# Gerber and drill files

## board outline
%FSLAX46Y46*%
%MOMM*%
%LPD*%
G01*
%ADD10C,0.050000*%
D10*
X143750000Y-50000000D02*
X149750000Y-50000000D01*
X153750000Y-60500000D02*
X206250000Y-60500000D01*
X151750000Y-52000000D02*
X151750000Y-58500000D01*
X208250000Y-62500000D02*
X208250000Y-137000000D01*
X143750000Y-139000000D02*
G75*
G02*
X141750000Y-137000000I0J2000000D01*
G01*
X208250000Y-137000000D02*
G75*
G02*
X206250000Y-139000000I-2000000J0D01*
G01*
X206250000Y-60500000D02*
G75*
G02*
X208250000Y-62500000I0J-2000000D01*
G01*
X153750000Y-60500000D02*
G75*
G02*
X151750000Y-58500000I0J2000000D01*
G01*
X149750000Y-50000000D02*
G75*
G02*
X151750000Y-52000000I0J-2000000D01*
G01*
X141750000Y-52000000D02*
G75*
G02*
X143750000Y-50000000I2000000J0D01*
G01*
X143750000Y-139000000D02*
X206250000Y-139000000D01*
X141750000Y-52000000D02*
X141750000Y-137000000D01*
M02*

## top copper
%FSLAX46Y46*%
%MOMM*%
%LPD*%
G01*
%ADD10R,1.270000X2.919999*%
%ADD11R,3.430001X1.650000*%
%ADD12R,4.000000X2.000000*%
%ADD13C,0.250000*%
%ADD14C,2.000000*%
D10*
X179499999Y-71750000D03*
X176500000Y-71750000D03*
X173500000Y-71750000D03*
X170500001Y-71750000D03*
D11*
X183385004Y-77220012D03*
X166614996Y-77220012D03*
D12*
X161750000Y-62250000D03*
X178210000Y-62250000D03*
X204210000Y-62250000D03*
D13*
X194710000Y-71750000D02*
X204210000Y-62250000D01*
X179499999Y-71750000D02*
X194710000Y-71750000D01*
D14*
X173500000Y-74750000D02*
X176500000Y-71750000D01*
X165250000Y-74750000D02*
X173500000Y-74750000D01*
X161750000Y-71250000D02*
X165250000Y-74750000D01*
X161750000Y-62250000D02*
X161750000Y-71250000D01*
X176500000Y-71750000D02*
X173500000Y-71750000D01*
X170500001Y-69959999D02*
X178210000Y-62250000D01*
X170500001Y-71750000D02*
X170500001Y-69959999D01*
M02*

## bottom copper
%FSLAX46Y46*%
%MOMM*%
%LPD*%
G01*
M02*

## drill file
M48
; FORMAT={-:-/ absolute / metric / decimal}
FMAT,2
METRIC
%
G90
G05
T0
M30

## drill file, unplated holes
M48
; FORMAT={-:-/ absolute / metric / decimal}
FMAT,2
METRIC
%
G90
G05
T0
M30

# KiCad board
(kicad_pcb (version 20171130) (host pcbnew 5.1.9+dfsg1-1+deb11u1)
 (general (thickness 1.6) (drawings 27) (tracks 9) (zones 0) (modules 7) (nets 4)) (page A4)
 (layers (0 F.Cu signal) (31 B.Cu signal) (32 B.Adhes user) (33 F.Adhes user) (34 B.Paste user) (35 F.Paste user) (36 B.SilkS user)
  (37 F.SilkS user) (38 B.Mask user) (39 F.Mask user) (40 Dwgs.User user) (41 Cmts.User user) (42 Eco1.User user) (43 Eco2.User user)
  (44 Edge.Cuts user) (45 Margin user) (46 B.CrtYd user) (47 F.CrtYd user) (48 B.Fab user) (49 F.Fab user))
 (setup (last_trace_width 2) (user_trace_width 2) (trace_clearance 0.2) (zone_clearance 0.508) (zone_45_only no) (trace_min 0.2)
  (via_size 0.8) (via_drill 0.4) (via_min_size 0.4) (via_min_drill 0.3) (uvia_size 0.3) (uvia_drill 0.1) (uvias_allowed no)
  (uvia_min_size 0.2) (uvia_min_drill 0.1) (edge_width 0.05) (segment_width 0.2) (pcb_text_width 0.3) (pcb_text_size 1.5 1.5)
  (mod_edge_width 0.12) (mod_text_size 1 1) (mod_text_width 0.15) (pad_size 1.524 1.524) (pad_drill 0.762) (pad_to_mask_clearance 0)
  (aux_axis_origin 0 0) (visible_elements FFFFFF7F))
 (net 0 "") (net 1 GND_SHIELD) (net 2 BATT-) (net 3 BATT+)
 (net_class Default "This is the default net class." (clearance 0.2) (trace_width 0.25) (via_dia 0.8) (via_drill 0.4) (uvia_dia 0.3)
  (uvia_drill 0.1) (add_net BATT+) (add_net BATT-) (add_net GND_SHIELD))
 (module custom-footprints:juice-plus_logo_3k (layer B.Cu) (at 198.25 133 180)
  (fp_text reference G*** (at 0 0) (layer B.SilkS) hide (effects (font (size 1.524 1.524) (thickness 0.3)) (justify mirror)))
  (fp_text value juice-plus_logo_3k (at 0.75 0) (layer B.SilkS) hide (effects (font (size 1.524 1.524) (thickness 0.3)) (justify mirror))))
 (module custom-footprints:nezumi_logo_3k (layer F.Cu) (at 146.5 55.5)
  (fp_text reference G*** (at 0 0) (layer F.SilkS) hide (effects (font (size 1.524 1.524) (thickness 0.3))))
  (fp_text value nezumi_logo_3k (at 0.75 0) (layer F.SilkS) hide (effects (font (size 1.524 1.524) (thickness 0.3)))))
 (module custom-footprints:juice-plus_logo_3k (layer F.Cu) (at 152 132)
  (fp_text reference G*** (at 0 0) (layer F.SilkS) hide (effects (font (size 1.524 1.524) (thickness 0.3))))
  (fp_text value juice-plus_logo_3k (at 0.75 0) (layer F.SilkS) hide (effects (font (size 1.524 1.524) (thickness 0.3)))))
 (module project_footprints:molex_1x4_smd (layer F.Cu) (at 175 76.87)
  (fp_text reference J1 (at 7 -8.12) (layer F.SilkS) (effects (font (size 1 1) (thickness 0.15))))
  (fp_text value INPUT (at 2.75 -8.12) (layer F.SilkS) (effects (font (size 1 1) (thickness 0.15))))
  (pad 1 smd rect (at 4.499999 -5.12) (size 1.27 2.919999) (layers F.Cu F.Paste F.Mask) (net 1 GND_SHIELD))
  (pad 2 smd rect (at 1.5 -5.12) (size 1.27 2.919999) (layers F.Cu F.Paste F.Mask) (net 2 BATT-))
  (pad 3 smd rect (at -1.5 -5.12) (size 1.27 2.919999) (layers F.Cu F.Paste F.Mask) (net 2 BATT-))
  (pad 4 smd rect (at -4.499999 -5.12) (size 1.27 2.919999) (layers F.Cu F.Paste F.Mask) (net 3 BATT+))
  (pad P1 smd rect (at 8.385004 0.350012) (size 3.430001 1.65) (layers F.Cu F.Paste F.Mask))
  (pad P2 smd rect (at -8.385004 0.350012) (size 3.430001 1.65) (layers F.Cu F.Paste F.Mask)))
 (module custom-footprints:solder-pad (layer F.Cu) (at 164.29 62.25 90)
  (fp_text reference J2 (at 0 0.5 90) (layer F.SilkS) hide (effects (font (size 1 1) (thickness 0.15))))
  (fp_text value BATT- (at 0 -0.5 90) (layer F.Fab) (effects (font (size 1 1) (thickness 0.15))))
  (pad 1 smd rect (at 0 -2.54 90) (size 2 4) (layers F.Cu F.Paste F.Mask) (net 2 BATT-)))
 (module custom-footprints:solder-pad (layer F.Cu) (at 180.75 62.25 90)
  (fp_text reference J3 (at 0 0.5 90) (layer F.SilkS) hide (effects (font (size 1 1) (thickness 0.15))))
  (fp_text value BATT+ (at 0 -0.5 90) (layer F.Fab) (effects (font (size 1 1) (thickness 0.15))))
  (pad 1 smd rect (at 0 -2.54 90) (size 2 4) (layers F.Cu F.Paste F.Mask) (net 3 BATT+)))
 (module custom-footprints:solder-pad (layer F.Cu) (at 206.75 62.25 90)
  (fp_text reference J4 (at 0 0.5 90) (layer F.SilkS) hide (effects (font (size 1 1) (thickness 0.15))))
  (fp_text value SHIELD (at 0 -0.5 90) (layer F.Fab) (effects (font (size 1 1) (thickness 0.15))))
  (pad 1 smd rect (at 0 -2.54 90) (size 2 4) (layers F.Cu F.Paste F.Mask) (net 1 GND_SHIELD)))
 (gr_line (start 143.75 50) (end 149.75 50) (layer Edge.Cuts) (width 0.05))
 (gr_line (start 153.75 60.5) (end 206.25 60.5) (layer Edge.Cuts) (width 0.05))
 (gr_line (start 151.75 52) (end 151.75 58.5) (layer Edge.Cuts) (width 0.05))
 (gr_line (start 208.25 62.5) (end 208.25 137) (layer Edge.Cuts) (width 0.05))
 (gr_arc (start 143.75 137) (end 141.75 137) (angle -90) (layer Edge.Cuts) (width 0.05))
 (gr_arc (start 206.25 137) (end 206.25 139) (angle -90) (layer Edge.Cuts) (width 0.05))
 (gr_arc (start 206.25 62.5) (end 208.25 62.5) (angle -90) (layer Edge.Cuts) (width 0.05))
 (gr_arc (start 153.75 58.5) (end 151.75 58.5) (angle -90) (layer Edge.Cuts) (width 0.05))
 (gr_arc (start 149.75 52) (end 151.75 52) (angle -90) (layer Edge.Cuts) (width 0.05))
 (gr_arc (start 143.75 52) (end 143.75 50) (angle -90) (layer Edge.Cuts) (width 0.05))
 (gr_line (start 143.75 139) (end 206.25 139) (layer Edge.Cuts) (width 0.05))
 (gr_line (start 141.75 52) (end 141.75 137) (layer Edge.Cuts) (width 0.05))
 (segment (start 194.71 71.75) (end 204.21 62.25) (width 0.25) (layer F.Cu) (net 1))
 (segment (start 179.499999 71.75) (end 194.71 71.75) (width 0.25) (layer F.Cu) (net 1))
 (segment (start 173.5 74.75) (end 176.5 71.75) (width 2) (layer F.Cu) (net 2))
 (segment (start 165.25 74.75) (end 173.5 74.75) (width 2) (layer F.Cu) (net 2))
 (segment (start 161.75 71.25) (end 165.25 74.75) (width 2) (layer F.Cu) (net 2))
 (segment (start 161.75 62.25) (end 161.75 71.25) (width 2) (layer F.Cu) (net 2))
 (segment (start 176.5 71.75) (end 173.5 71.75) (width 2) (layer F.Cu) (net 2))
 (segment (start 170.500001 69.959999) (end 178.21 62.25) (width 2) (layer F.Cu) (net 3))
 (segment (start 170.500001 71.75) (end 170.500001 69.959999) (width 2) (layer F.Cu) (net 3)))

